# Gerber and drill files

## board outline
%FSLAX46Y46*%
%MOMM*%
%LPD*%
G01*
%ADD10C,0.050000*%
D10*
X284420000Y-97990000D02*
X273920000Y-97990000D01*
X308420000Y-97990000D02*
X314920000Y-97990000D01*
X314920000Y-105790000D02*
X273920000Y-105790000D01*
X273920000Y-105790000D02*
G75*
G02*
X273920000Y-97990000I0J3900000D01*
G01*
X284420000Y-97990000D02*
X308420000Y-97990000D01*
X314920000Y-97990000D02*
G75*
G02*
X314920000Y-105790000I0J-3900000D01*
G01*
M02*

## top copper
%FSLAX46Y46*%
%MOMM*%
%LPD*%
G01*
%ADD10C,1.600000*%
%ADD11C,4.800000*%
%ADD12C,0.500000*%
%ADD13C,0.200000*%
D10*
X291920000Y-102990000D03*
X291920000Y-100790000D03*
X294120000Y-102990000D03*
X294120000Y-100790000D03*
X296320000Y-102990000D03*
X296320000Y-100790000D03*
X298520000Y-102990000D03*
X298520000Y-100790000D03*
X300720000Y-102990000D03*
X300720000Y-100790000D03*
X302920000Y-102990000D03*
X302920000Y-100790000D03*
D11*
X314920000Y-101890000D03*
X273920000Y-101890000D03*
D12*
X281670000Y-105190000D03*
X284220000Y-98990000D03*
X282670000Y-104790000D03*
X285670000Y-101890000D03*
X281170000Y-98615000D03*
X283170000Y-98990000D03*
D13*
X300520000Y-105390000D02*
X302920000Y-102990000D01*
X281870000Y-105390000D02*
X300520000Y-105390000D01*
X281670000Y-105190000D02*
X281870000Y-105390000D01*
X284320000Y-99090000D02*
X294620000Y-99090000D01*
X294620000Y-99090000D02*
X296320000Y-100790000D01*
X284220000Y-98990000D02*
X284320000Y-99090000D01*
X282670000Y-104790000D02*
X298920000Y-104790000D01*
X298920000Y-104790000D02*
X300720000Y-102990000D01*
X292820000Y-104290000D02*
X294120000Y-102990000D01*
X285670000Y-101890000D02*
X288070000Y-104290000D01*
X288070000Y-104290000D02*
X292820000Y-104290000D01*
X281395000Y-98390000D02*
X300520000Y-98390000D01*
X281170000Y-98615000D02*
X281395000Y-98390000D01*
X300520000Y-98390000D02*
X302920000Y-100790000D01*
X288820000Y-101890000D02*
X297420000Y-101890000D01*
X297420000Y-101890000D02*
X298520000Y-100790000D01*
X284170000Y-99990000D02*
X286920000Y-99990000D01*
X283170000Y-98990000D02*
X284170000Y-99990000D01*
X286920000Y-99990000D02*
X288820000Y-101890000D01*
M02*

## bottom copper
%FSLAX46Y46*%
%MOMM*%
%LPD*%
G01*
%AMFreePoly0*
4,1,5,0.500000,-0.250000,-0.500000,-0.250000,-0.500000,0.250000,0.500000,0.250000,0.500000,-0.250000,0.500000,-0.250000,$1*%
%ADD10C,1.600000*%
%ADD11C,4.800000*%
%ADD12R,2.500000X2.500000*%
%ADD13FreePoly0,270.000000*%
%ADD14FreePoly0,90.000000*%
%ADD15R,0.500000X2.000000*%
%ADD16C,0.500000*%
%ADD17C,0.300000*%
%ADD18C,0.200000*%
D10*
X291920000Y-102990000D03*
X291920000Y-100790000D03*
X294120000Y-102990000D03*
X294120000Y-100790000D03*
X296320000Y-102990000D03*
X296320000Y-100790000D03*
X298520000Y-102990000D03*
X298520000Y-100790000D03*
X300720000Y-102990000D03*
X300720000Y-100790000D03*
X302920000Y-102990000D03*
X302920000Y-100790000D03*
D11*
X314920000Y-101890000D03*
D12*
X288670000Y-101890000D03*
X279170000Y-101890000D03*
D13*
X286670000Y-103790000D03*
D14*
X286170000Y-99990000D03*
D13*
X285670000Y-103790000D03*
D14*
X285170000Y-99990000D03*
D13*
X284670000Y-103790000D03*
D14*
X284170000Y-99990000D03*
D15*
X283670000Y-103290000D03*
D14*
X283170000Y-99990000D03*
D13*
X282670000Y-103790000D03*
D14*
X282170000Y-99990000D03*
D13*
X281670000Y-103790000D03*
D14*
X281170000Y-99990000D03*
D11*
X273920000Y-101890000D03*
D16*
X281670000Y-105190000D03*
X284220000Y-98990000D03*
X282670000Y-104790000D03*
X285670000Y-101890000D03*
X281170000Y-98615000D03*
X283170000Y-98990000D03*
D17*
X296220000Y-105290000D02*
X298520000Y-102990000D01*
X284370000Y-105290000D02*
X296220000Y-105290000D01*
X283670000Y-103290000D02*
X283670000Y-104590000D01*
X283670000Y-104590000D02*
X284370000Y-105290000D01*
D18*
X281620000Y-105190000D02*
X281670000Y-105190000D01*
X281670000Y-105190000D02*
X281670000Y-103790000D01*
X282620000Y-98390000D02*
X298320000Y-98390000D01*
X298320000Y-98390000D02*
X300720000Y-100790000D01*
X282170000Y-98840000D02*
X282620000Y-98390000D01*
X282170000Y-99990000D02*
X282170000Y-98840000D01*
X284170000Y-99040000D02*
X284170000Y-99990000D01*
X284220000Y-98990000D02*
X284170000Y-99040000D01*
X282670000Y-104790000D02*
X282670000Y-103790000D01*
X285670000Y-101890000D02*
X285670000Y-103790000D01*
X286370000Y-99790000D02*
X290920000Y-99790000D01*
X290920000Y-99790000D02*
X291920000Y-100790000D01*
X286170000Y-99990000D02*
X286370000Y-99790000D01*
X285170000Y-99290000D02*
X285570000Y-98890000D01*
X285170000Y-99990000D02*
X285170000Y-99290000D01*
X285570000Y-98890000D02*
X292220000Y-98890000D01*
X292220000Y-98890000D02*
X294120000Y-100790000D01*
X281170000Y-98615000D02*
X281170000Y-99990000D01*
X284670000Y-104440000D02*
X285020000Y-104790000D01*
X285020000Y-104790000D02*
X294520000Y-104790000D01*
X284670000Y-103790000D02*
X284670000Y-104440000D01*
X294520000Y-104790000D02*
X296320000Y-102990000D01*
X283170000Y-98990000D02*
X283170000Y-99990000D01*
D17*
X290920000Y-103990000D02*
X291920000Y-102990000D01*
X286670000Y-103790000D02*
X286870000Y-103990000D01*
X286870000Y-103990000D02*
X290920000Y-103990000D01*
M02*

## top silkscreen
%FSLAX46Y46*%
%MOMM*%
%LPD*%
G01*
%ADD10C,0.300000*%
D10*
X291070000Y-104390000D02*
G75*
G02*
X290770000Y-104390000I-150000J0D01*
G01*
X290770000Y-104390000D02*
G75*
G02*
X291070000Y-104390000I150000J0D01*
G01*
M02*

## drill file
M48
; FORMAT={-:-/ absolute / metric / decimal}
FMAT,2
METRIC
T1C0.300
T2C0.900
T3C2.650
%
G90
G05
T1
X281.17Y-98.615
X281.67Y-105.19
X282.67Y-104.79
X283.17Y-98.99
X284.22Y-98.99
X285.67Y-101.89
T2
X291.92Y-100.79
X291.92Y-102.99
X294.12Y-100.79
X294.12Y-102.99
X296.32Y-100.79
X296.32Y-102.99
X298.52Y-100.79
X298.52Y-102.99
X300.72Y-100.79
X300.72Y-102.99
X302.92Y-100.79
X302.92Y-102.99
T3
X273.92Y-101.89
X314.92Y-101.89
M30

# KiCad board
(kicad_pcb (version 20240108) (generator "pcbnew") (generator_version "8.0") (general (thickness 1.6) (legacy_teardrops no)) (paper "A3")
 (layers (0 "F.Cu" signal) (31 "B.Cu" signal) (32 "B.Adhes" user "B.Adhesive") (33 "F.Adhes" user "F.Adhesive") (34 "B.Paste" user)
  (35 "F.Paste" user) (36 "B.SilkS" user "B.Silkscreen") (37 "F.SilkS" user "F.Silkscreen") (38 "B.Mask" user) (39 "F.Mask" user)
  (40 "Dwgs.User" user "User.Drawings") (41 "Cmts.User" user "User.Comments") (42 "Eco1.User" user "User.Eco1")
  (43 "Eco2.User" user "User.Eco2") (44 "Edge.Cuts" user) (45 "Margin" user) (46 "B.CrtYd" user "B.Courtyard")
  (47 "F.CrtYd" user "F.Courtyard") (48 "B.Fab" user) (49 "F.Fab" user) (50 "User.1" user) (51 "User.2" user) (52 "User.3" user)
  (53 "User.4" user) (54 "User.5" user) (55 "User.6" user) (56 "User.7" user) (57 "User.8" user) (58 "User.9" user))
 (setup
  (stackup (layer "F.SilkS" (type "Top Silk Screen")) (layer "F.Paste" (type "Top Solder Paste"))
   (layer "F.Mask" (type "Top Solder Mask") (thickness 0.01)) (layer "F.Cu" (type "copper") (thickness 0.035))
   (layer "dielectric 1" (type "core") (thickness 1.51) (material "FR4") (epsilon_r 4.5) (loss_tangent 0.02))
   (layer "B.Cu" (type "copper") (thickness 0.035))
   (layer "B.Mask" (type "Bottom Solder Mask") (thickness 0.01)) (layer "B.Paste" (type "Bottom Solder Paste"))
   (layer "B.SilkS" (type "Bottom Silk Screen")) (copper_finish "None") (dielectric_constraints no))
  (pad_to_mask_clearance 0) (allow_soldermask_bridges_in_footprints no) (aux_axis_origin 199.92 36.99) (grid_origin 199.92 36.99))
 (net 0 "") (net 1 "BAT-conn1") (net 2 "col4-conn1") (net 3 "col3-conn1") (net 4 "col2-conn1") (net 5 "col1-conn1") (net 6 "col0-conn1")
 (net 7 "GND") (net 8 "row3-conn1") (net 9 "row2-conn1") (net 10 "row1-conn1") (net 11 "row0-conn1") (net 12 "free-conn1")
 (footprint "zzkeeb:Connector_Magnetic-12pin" (layer "B.Cu") (at 297.42 101.89 90)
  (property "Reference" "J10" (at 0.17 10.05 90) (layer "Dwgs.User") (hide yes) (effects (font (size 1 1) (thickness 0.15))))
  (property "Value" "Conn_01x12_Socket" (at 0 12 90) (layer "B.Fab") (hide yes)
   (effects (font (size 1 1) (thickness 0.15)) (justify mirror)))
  (fp_circle (center -2.5 -6.5) (end -2.25 -6.5) (stroke (width 0.1) (type solid)) (fill solid) (layer "F.SilkS"))
  (pad "1" thru_hole circle (at -1.1 -5.5 270) (size 1.6 1.6) (drill 0.9) (layers "*.Cu" "*.Mask") (remove_unused_layers no)
   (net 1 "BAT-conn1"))
  (pad "2" thru_hole circle (at 1.1 -5.5 270) (size 1.6 1.6) (drill 0.9) (layers "*.Cu" "*.Mask") (remove_unused_layers no)
   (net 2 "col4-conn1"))
  (pad "3" thru_hole circle (at -1.1 -3.3 270) (size 1.6 1.6) (drill 0.9) (layers "*.Cu" "*.Mask") (remove_unused_layers no)
   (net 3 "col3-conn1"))
  (pad "4" thru_hole circle (at 1.1 -3.3 270) (size 1.6 1.6) (drill 0.9) (layers "*.Cu" "*.Mask") (remove_unused_layers no)
   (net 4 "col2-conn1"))
  (pad "5" thru_hole circle (at -1.1 -1.1 270) (size 1.6 1.6) (drill 0.9) (layers "*.Cu" "*.Mask") (remove_unused_layers no)
   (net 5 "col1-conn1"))
  (pad "6" thru_hole circle (at 1.1 -1.1 270) (size 1.6 1.6) (drill 0.9) (layers "*.Cu" "*.Mask") (remove_unused_layers no)
   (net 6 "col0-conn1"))
  (pad "7" thru_hole circle (at -1.1 1.1 270) (size 1.6 1.6) (drill 0.9) (layers "*.Cu" "*.Mask") (remove_unused_layers no) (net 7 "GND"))
  (pad "8" thru_hole circle (at 1.1 1.1 270) (size 1.6 1.6) (drill 0.9) (layers "*.Cu" "*.Mask") (remove_unused_layers no)
   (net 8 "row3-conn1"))
  (pad "9" thru_hole circle (at -1.1 3.3 270) (size 1.6 1.6) (drill 0.9) (layers "*.Cu" "*.Mask") (remove_unused_layers no)
   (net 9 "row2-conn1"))
  (pad "10" thru_hole circle (at 1.1 3.3 270) (size 1.6 1.6) (drill 0.9) (layers "*.Cu" "*.Mask") (remove_unused_layers no)
   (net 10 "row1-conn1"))
  (pad "11" thru_hole circle (at -1.1 5.5 270) (size 1.6 1.6) (drill 0.9) (layers "*.Cu" "*.Mask") (remove_unused_layers no)
   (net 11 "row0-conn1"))
  (pad "12" thru_hole circle (at 1.1 5.5 270) (size 1.6 1.6) (drill 0.9) (layers "*.Cu" "*.Mask") (remove_unused_layers no)
   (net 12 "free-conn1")))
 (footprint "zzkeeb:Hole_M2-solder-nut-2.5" (layer "B.Cu") (at 314.92 101.89 90)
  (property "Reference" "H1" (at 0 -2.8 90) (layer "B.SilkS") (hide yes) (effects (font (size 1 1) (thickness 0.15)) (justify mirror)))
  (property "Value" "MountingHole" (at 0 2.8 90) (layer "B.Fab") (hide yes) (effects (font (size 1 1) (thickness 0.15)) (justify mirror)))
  (pad "" thru_hole circle (at 0 0 90) (size 4.8 4.8) (drill 2.65) (layers "*.Cu" "B.Mask") (remove_unused_layers no)))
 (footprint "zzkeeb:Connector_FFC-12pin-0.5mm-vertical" (layer "B.Cu") (at 283.92 101.89 180)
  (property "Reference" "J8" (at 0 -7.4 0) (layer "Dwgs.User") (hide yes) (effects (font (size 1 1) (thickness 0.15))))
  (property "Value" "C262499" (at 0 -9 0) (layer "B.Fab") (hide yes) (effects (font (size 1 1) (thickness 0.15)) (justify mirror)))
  (pad "" smd rect (at -4.75 0 90) (size 2.5 2.5) (layers "B.Cu" "B.Paste" "B.Mask"))
  (pad "" smd rect (at 4.75 0 90) (size 2.5 2.5) (layers "B.Cu" "B.Paste" "B.Mask"))
  (pad "1" smd custom (at -2.75 -1.9 270) (size 1 0.5) (layers "B.Cu" "B.Paste" "B.Mask") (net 1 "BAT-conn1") (thermal_bridge_angle 45)
   (options (clearance outline) (anchor rect)) (primitives))
  (pad "2" smd custom (at -2.25 1.9 90) (size 1 0.5) (layers "B.Cu" "B.Paste" "B.Mask") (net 2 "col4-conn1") (thermal_bridge_angle 45)
   (options (clearance outline) (anchor rect)) (primitives))
  (pad "3" smd custom (at -1.75 -1.9 270) (size 1 0.5) (layers "B.Cu" "B.Paste" "B.Mask") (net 3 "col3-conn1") (thermal_bridge_angle 45)
   (options (clearance outline) (anchor rect)) (primitives))
  (pad "4" smd custom (at -1.25 1.9 90) (size 1 0.5) (layers "B.Cu" "B.Paste" "B.Mask") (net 4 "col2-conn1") (thermal_bridge_angle 45)
   (options (clearance outline) (anchor rect)) (primitives))
  (pad "5" smd custom (at -0.75 -1.9 270) (size 1 0.5) (layers "B.Cu" "B.Paste" "B.Mask") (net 5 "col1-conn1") (thermal_bridge_angle 45)
   (options (clearance outline) (anchor rect)) (primitives))
  (pad "6" smd custom (at -0.25 1.9 90) (size 1 0.5) (layers "B.Cu" "B.Paste" "B.Mask") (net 6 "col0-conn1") (thermal_bridge_angle 45)
   (options (clearance outline) (anchor rect)) (primitives))
  (pad "7" smd rect (at 0.25 -1.4 180) (size 0.5 2) (layers "B.Cu" "B.Paste" "B.Mask") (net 7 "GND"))
  (pad "8" smd custom (at 0.75 1.9 90) (size 1 0.5) (layers "B.Cu" "B.Paste" "B.Mask") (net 8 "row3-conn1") (thermal_bridge_angle 45)
   (options (clearance outline) (anchor rect)) (primitives))
  (pad "9" smd custom (at 1.25 -1.9 270) (size 1 0.5) (layers "B.Cu" "B.Paste" "B.Mask") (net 9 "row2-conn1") (thermal_bridge_angle 45)
   (options (clearance outline) (anchor rect)) (primitives))
  (pad "10" smd custom (at 1.75 1.9 90) (size 1 0.5) (layers "B.Cu" "B.Paste" "B.Mask") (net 10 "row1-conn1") (thermal_bridge_angle 45)
   (options (clearance outline) (anchor rect)) (primitives))
  (pad "11" smd custom (at 2.25 -1.9 270) (size 1 0.5) (layers "B.Cu" "B.Paste" "B.Mask") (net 11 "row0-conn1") (thermal_bridge_angle 45)
   (options (clearance outline) (anchor rect)) (primitives))
  (pad "12" smd custom (at 2.75 1.9 90) (size 1 0.5) (layers "B.Cu" "B.Paste" "B.Mask") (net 12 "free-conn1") (thermal_bridge_angle 45)
   (options (clearance outline) (anchor rect)) (primitives)))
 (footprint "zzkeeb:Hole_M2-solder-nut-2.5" (layer "B.Cu") (at 273.92 101.89 90)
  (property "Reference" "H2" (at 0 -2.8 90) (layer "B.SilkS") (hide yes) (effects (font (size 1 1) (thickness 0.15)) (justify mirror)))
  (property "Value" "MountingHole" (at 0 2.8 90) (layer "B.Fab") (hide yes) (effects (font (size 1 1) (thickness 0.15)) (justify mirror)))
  (pad "" thru_hole circle (at 0 0 90) (size 4.8 4.8) (drill 2.65) (layers "*.Cu" "B.Mask") (remove_unused_layers no)))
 (gr_line (start 284.42 97.99) (end 273.92 97.99) (stroke (width 0.05) (type default)) (layer "Edge.Cuts"))
 (gr_line (start 308.42 97.99) (end 314.92 97.99) (stroke (width 0.05) (type default)) (layer "Edge.Cuts"))
 (gr_line (start 314.92 105.79) (end 273.92 105.79) (stroke (width 0.05) (type default)) (layer "Edge.Cuts"))
 (gr_arc (start 273.92 105.79) (mid 270.02 101.89) (end 273.92 97.99) (stroke (width 0.05) (type default)) (layer "Edge.Cuts"))
 (gr_line (start 284.42 97.99) (end 308.42 97.99) (stroke (width 0.05) (type default)) (layer "Edge.Cuts"))
 (gr_arc (start 314.92 97.99) (mid 318.82 101.89) (end 314.92 105.79) (stroke (width 0.05) (type default)) (layer "Edge.Cuts"))
 (segment (start 296.22 105.29) (end 298.52 102.99) (width 0.3) (layer "B.Cu") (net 7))
 (segment (start 284.37 105.29) (end 296.22 105.29) (width 0.3) (layer "B.Cu") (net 7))
 (segment (start 283.67 103.29) (end 283.67 104.59) (width 0.3) (layer "B.Cu") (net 7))
 (segment (start 283.67 104.59) (end 284.37 105.29) (width 0.3) (layer "B.Cu") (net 7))
 (segment (start 300.52 105.39) (end 302.92 102.99) (width 0.2) (layer "F.Cu") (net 11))
 (segment (start 281.87 105.39) (end 300.52 105.39) (width 0.2) (layer "F.Cu") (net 11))
 (segment (start 281.67 105.19) (end 281.87 105.39) (width 0.2) (layer "F.Cu") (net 11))
 (via (at 281.67 105.19) (size 0.5) (drill 0.3) (layers "F.Cu" "B.Cu") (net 11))
 (segment (start 281.62 105.19) (end 281.67 105.19) (width 0.2) (layer "B.Cu") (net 11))
 (segment (start 281.67 105.19) (end 281.67 103.79) (width 0.2) (layer "B.Cu") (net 11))
 (segment (start 282.62 98.39) (end 298.32 98.39) (width 0.2) (layer "B.Cu") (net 10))
 (segment (start 298.32 98.39) (end 300.72 100.79) (width 0.2) (layer "B.Cu") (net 10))
 (segment (start 282.17 98.84) (end 282.62 98.39) (width 0.2) (layer "B.Cu") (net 10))
 (segment (start 282.17 99.99) (end 282.17 98.84) (width 0.2) (layer "B.Cu") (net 10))
 (segment (start 284.32 99.09) (end 294.62 99.09) (width 0.2) (layer "F.Cu") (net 6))
 (segment (start 294.62 99.09) (end 296.32 100.79) (width 0.2) (layer "F.Cu") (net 6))
 (segment (start 284.22 98.99) (end 284.32 99.09) (width 0.2) (layer "F.Cu") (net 6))
 (via (at 284.22 98.99) (size 0.5) (drill 0.3) (layers "F.Cu" "B.Cu") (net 6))
 (segment (start 284.17 99.04) (end 284.17 99.99) (width 0.2) (layer "B.Cu") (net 6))
 (segment (start 284.22 98.99) (end 284.17 99.04) (width 0.2) (layer "B.Cu") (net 6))
 (segment (start 282.67 104.79) (end 298.92 104.79) (width 0.2) (layer "F.Cu") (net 9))
 (segment (start 298.92 104.79) (end 300.72 102.99) (width 0.2) (layer "F.Cu") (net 9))
 (via (at 282.67 104.79) (size 0.5) (drill 0.3) (layers "F.Cu" "B.Cu") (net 9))
 (segment (start 282.67 104.79) (end 282.67 103.79) (width 0.2) (layer "B.Cu") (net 9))
 (segment (start 292.82 104.29) (end 294.12 102.99) (width 0.2) (layer "F.Cu") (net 3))
 (segment (start 285.67 101.89) (end 288.07 104.29) (width 0.2) (layer "F.Cu") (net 3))
 (segment (start 288.07 104.29) (end 292.82 104.29) (width 0.2) (layer "F.Cu") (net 3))
 (via (at 285.67 101.89) (size 0.5) (drill 0.3) (layers "F.Cu" "B.Cu") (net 3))
 (segment (start 285.67 101.89) (end 285.67 103.79) (width 0.2) (layer "B.Cu") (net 3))
 (segment (start 286.37 99.79) (end 290.92 99.79) (width 0.2) (layer "B.Cu") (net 2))
 (segment (start 290.92 99.79) (end 291.92 100.79) (width 0.2) (layer "B.Cu") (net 2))
 (segment (start 286.17 99.99) (end 286.37 99.79) (width 0.2) (layer "B.Cu") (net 2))
 (segment (start 285.17 99.29) (end 285.57 98.89) (width 0.2) (layer "B.Cu") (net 4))
 (segment (start 285.17 99.99) (end 285.17 99.29) (width 0.2) (layer "B.Cu") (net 4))
 (segment (start 285.57 98.89) (end 292.22 98.89) (width 0.2) (layer "B.Cu") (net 4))
 (segment (start 292.22 98.89) (end 294.12 100.79) (width 0.2) (layer "B.Cu") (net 4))
 (segment (start 281.395 98.39) (end 300.52 98.39) (width 0.2) (layer "F.Cu") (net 12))
 (segment (start 281.17 98.615) (end 281.395 98.39) (width 0.2) (layer "F.Cu") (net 12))
 (segment (start 300.52 98.39) (end 302.92 100.79) (width 0.2) (layer "F.Cu") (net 12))
 (via (at 281.17 98.615) (size 0.5) (drill 0.3) (layers "F.Cu" "B.Cu") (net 12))
 (segment (start 281.17 98.615) (end 281.17 99.99) (width 0.2) (layer "B.Cu") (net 12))
 (segment (start 284.67 104.44) (end 285.02 104.79) (width 0.2) (layer "B.Cu") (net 5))
 (segment (start 285.02 104.79) (end 294.52 104.79) (width 0.2) (layer "B.Cu") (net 5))
 (segment (start 284.67 103.79) (end 284.67 104.44) (width 0.2) (layer "B.Cu") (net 5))
 (segment (start 294.52 104.79) (end 296.32 102.99) (width 0.2) (layer "B.Cu") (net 5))
 (segment (start 288.82 101.89) (end 297.42 101.89) (width 0.2) (layer "F.Cu") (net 8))
 (segment (start 297.42 101.89) (end 298.52 100.79) (width 0.2) (layer "F.Cu") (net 8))
 (segment (start 284.17 99.99) (end 286.92 99.99) (width 0.2) (layer "F.Cu") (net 8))
 (segment (start 283.17 98.99) (end 284.17 99.99) (width 0.2) (layer "F.Cu") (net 8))
 (segment (start 286.92 99.99) (end 288.82 101.89) (width 0.2) (layer "F.Cu") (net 8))
 (via (at 283.17 98.99) (size 0.5) (drill 0.3) (layers "F.Cu" "B.Cu") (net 8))
 (segment (start 283.17 98.99) (end 283.17 99.99) (width 0.2) (layer "B.Cu") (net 8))
 (segment (start 290.92 103.99) (end 291.92 102.99) (width 0.3) (layer "B.Cu") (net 1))
 (segment (start 286.67 103.79) (end 286.87 103.99) (width 0.3) (layer "B.Cu") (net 1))
 (segment (start 286.87 103.99) (end 290.92 103.99) (width 0.3) (layer "B.Cu") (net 1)))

